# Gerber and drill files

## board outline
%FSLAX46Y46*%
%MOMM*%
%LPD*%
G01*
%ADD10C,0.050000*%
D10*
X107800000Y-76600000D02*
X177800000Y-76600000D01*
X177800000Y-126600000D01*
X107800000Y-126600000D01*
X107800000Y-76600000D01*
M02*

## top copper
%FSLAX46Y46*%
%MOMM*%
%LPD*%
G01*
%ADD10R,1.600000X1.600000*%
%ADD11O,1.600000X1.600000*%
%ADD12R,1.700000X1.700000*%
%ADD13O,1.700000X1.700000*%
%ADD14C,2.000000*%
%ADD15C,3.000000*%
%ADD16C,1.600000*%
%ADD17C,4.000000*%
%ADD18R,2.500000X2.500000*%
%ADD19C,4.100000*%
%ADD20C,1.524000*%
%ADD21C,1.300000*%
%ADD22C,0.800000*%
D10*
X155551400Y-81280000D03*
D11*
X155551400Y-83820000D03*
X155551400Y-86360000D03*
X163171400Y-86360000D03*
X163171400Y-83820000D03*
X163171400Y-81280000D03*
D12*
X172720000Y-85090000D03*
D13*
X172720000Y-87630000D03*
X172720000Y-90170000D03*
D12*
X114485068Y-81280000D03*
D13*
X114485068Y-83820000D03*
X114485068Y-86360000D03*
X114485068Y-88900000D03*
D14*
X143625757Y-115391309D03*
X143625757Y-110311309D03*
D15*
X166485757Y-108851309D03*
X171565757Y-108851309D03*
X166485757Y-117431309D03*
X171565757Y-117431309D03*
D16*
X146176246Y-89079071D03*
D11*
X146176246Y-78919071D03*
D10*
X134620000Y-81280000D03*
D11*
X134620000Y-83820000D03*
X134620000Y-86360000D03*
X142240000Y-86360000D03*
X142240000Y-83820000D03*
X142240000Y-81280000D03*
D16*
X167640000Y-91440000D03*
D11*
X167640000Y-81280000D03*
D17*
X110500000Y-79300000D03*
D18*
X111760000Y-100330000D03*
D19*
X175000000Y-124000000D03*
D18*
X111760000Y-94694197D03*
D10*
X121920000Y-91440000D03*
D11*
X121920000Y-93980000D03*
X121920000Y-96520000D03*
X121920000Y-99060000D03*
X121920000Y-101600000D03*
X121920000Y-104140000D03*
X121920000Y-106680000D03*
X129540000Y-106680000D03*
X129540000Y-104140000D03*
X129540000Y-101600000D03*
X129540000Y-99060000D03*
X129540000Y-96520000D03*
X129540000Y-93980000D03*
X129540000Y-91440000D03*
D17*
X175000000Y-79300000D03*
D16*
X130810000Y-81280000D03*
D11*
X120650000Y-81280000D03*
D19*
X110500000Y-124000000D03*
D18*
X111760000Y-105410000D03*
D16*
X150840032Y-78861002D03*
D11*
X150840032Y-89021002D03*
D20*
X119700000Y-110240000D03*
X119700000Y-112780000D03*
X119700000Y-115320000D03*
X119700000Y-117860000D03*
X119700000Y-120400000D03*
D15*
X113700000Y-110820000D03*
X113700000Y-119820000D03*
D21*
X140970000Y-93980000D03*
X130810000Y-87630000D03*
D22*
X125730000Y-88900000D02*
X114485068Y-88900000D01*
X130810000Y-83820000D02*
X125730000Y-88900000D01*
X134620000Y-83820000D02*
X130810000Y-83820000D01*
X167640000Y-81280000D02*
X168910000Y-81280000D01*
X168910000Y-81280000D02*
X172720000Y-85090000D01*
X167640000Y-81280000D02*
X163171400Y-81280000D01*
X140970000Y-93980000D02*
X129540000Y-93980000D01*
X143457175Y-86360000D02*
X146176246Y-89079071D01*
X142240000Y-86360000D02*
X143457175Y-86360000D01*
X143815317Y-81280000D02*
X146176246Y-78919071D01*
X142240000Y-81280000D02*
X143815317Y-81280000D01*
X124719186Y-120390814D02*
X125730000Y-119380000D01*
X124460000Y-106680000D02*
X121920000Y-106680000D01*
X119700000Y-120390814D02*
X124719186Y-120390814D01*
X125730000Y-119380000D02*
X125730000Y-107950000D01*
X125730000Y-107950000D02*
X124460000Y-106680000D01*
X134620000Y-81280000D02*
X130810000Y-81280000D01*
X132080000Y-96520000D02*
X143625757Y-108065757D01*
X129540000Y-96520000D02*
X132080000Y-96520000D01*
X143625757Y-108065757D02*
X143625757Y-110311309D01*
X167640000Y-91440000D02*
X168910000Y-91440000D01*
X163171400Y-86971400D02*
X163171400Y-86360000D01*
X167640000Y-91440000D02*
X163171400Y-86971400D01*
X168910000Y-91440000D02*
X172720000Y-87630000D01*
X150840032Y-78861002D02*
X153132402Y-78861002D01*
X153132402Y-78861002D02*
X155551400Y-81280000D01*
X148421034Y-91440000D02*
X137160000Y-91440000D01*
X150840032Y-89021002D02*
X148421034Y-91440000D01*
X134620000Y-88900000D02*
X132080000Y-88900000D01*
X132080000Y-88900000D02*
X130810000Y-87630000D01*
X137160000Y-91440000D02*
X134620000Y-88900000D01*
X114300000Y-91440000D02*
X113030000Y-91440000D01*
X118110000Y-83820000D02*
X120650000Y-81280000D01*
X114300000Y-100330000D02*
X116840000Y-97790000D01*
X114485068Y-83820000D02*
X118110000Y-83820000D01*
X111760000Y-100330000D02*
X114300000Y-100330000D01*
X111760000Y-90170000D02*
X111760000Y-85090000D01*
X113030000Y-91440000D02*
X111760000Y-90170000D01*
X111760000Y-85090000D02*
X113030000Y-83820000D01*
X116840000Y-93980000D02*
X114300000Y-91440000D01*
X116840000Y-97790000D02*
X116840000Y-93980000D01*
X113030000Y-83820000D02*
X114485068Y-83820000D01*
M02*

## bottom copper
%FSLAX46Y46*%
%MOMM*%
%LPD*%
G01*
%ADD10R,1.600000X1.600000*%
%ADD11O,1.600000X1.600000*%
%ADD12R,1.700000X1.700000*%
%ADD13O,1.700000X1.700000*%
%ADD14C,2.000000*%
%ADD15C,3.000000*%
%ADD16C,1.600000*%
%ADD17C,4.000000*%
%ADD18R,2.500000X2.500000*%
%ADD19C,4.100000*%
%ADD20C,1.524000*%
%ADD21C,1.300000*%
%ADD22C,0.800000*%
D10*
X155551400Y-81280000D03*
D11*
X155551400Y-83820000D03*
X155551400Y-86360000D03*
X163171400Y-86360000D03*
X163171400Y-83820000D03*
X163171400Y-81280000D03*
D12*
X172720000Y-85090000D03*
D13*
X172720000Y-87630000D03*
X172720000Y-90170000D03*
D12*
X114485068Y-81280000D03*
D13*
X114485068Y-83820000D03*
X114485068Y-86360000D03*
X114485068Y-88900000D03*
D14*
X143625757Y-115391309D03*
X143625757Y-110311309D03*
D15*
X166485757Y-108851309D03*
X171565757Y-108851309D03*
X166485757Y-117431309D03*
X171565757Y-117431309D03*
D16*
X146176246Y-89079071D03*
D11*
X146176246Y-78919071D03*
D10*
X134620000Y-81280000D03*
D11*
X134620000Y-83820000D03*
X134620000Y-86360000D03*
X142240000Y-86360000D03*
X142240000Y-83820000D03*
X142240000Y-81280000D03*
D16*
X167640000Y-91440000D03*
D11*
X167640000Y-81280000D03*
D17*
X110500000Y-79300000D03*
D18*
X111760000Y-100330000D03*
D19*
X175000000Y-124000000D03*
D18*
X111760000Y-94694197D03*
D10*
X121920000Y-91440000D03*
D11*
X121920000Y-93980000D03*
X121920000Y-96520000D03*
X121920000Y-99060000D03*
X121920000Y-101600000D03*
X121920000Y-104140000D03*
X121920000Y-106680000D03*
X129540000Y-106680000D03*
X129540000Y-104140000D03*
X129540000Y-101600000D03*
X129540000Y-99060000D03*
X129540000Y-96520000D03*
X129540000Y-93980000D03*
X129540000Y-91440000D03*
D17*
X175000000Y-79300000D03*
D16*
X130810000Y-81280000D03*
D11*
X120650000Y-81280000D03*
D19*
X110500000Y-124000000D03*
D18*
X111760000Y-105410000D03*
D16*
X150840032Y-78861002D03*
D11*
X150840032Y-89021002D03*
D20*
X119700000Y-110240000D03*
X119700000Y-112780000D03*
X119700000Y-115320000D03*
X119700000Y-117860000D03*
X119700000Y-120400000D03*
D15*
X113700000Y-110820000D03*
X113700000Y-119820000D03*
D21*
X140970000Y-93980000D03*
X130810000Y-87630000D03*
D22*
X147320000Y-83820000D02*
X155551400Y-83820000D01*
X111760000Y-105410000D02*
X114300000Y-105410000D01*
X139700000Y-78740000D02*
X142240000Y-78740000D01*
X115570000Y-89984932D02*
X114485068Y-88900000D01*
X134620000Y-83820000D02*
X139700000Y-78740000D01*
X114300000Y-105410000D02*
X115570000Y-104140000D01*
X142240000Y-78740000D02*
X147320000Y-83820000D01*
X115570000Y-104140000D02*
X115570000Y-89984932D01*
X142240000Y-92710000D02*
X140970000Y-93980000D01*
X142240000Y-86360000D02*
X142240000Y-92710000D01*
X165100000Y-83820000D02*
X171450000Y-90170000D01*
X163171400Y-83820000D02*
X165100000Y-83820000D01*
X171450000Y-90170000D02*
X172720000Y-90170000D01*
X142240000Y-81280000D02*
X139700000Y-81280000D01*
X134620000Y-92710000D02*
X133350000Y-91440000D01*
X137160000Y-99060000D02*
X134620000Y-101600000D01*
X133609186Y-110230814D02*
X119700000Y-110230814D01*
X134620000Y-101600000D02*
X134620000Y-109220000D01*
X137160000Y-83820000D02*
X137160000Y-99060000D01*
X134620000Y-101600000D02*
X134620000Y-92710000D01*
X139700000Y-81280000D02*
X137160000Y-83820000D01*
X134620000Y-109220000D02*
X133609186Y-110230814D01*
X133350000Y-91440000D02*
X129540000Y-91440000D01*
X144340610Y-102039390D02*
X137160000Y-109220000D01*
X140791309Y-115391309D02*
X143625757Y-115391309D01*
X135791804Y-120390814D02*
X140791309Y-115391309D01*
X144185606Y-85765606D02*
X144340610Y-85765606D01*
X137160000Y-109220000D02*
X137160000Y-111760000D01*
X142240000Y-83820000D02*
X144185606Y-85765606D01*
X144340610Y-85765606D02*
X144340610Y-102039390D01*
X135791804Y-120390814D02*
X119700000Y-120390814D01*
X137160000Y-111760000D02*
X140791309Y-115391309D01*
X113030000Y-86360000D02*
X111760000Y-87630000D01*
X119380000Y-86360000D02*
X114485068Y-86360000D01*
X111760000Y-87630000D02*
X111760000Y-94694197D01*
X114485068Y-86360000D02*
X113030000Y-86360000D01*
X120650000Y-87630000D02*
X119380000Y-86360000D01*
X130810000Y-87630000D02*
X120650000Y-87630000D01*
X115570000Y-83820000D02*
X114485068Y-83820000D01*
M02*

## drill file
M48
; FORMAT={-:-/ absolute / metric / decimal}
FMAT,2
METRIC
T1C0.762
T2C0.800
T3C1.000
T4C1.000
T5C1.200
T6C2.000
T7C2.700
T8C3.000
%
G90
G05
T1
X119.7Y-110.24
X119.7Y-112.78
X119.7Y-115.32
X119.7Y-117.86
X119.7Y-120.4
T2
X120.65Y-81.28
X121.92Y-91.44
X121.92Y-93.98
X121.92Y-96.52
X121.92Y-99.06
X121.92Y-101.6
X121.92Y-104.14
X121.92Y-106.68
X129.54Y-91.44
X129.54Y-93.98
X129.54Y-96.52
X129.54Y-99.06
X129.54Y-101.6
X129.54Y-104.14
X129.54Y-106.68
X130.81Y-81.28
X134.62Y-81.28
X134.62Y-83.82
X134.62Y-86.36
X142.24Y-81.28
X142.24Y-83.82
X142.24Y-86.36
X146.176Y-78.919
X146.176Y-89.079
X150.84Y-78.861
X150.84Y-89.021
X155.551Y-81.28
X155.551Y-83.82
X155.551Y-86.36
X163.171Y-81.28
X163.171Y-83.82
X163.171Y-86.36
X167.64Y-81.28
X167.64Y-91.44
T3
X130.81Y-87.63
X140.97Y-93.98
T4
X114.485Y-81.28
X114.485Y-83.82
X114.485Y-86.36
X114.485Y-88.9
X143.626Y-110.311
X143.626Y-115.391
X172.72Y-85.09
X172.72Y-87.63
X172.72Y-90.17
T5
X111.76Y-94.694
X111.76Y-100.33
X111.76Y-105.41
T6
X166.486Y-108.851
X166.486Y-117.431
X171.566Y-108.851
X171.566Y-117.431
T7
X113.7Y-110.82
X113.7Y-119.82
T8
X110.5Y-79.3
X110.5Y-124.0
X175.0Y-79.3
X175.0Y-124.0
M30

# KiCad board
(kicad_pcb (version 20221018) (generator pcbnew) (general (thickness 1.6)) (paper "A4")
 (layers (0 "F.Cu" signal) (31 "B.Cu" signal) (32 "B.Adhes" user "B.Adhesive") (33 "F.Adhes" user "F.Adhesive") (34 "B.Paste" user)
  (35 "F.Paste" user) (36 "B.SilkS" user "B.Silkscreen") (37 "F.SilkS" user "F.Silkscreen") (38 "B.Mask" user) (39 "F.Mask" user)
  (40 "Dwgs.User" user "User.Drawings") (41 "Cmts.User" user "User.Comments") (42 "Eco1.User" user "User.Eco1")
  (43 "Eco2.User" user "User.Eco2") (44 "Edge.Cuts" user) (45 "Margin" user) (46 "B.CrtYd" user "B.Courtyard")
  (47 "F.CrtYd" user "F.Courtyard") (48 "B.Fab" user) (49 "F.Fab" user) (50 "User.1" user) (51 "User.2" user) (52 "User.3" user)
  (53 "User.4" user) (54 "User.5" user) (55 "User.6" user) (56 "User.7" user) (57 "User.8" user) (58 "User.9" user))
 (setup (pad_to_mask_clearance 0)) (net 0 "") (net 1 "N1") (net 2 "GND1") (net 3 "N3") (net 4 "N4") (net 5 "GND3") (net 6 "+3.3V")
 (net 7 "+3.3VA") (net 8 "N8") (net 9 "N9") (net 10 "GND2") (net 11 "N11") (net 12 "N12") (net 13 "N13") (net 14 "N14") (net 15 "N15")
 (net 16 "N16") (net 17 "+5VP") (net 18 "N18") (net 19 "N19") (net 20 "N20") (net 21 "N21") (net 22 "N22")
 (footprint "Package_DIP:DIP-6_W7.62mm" (layer "F.Cu") (at 155.5514 81.28)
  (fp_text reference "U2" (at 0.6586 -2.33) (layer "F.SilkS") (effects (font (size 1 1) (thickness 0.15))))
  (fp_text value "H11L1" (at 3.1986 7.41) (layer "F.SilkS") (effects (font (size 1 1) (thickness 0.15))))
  (pad "1" thru_hole rect (at 0 0) (size 1.6 1.6) (drill 0.8) (layers "*.Cu" "*.Mask") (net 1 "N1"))
  (pad "2" thru_hole oval (at 0 2.54) (size 1.6 1.6) (drill 0.8) (layers "*.Cu" "*.Mask") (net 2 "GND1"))
  (pad "3" thru_hole oval (at 0 5.08) (size 1.6 1.6) (drill 0.8) (layers "*.Cu" "*.Mask") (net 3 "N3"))
  (pad "4" thru_hole oval (at 7.62 5.08) (size 1.6 1.6) (drill 0.8) (layers "*.Cu" "*.Mask") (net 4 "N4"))
  (pad "5" thru_hole oval (at 7.62 2.54) (size 1.6 1.6) (drill 0.8) (layers "*.Cu" "*.Mask") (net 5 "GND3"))
  (pad "6" thru_hole oval (at 7.62 0) (size 1.6 1.6) (drill 0.8) (layers "*.Cu" "*.Mask") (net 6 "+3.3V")))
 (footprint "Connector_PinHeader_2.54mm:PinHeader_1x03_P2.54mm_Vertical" (layer "F.Cu") (at 172.72 85.09)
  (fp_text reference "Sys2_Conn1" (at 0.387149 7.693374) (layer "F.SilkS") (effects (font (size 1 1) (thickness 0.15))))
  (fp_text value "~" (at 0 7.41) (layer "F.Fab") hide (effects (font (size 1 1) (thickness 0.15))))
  (pad "1" thru_hole rect (at 0 0) (size 1.7 1.7) (drill 1) (layers "*.Cu" "*.Mask") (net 6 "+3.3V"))
  (pad "2" thru_hole oval (at 0 2.54) (size 1.7 1.7) (drill 1) (layers "*.Cu" "*.Mask") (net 4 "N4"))
  (pad "3" thru_hole oval (at 0 5.08) (size 1.7 1.7) (drill 1) (layers "*.Cu" "*.Mask") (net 5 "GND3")))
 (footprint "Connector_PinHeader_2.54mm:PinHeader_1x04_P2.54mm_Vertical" (layer "F.Cu") (at 114.485068 81.28)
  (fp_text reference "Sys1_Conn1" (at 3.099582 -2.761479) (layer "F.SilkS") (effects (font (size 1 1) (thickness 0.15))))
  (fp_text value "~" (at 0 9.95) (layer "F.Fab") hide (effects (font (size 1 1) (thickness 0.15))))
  (pad "1" thru_hole rect (at 0 0) (size 1.7 1.7) (drill 1) (layers "*.Cu" "*.Mask") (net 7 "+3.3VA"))
  (pad "2" thru_hole oval (at 0 2.54) (size 1.7 1.7) (drill 1) (layers "*.Cu" "*.Mask") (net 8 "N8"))
  (pad "3" thru_hole oval (at 0 5.08) (size 1.7 1.7) (drill 1) (layers "*.Cu" "*.Mask") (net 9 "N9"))
  (pad "4" thru_hole oval (at 0 7.62) (size 1.7 1.7) (drill 1) (layers "*.Cu" "*.Mask") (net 2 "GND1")))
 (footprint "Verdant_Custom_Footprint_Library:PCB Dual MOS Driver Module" (layer "F.Cu") (at 148.705757 112.851309)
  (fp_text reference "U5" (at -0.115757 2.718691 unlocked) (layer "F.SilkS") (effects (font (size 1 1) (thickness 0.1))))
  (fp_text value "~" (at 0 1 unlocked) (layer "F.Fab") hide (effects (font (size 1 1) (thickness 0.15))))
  (pad "1" thru_hole circle (at -5.08 2.54) (size 2 2) (drill 1) (layers "*.Cu" "*.Mask") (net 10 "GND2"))
  (pad "2" thru_hole circle (at -5.08 -2.54) (size 2 2) (drill 1) (layers "*.Cu" "*.Mask") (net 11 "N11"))
  (pad "3" thru_hole circle (at 17.78 -4 90) (size 3 3) (drill 2) (layers "*.Cu" "*.Mask") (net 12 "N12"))
  (pad "4" thru_hole circle (at 22.86 -4) (size 3 3) (drill 2) (layers "*.Cu" "*.Mask") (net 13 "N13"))
  (pad "5" thru_hole circle (at 17.78 4.58) (size 3 3) (drill 2) (layers "*.Cu" "*.Mask") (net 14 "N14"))
  (pad "6" thru_hole circle (at 22.86 4.58) (size 3 3) (drill 2) (layers "*.Cu" "*.Mask") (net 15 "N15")))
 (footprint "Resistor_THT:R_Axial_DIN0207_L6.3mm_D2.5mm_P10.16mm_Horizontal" (layer "F.Cu") (at 146.176246 89.079071 90)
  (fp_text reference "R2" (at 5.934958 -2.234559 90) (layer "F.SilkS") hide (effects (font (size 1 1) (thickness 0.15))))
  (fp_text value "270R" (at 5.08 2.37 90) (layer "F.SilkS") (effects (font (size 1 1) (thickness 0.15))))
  (pad "1" thru_hole circle (at 0 0 90) (size 1.6 1.6) (drill 0.8) (layers "*.Cu" "*.Mask") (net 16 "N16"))
  (pad "2" thru_hole oval (at 10.16 0 90) (size 1.6 1.6) (drill 0.8) (layers "*.Cu" "*.Mask") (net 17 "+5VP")))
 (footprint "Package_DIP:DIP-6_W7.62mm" (layer "F.Cu") (at 134.62 81.28)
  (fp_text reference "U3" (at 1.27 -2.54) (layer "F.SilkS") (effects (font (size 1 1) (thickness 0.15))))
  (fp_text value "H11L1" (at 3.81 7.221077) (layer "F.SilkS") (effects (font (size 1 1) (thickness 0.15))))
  (pad "1" thru_hole rect (at 0 0) (size 1.6 1.6) (drill 0.8) (layers "*.Cu" "*.Mask") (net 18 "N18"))
  (pad "2" thru_hole oval (at 0 2.54) (size 1.6 1.6) (drill 0.8) (layers "*.Cu" "*.Mask") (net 2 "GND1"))
  (pad "3" thru_hole oval (at 0 5.08) (size 1.6 1.6) (drill 0.8) (layers "*.Cu" "*.Mask") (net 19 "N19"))
  (pad "4" thru_hole oval (at 7.62 5.08) (size 1.6 1.6) (drill 0.8) (layers "*.Cu" "*.Mask") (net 16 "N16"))
  (pad "5" thru_hole oval (at 7.62 2.54) (size 1.6 1.6) (drill 0.8) (layers "*.Cu" "*.Mask") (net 10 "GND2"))
  (pad "6" thru_hole oval (at 7.62 0) (size 1.6 1.6) (drill 0.8) (layers "*.Cu" "*.Mask") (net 17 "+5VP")))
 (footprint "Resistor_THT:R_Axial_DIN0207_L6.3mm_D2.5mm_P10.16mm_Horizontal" (layer "F.Cu") (at 167.64 91.44 90)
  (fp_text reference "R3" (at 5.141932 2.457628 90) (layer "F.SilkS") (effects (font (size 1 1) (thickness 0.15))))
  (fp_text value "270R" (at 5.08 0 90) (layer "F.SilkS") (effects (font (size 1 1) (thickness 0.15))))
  (pad "1" thru_hole circle (at 0 0 90) (size 1.6 1.6) (drill 0.8) (layers "*.Cu" "*.Mask") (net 4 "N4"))
  (pad "2" thru_hole oval (at 10.16 0 90) (size 1.6 1.6) (drill 0.8) (layers "*.Cu" "*.Mask") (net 6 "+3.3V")))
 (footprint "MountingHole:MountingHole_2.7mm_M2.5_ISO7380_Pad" (layer "F.Cu") (at 110.5 79.3)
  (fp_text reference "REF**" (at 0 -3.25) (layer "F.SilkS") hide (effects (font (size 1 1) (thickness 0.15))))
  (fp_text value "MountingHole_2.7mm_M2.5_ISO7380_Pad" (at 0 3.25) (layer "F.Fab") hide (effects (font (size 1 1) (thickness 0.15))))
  (pad "1" thru_hole circle (at 0 0) (size 4 4) (drill 3) (layers "*.Cu" "*.Mask")))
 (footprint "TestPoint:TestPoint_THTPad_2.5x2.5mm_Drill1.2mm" (layer "F.Cu") (at 111.76 100.33)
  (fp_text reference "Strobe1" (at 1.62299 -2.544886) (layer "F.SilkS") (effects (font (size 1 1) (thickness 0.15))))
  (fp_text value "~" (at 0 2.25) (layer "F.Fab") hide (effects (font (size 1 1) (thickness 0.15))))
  (pad "1" thru_hole rect (at 0 0) (size 2.5 2.5) (drill 1.2) (layers "*.Cu" "*.Mask") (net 8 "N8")))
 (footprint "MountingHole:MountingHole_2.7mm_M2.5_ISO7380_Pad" (layer "F.Cu") (at 175 124)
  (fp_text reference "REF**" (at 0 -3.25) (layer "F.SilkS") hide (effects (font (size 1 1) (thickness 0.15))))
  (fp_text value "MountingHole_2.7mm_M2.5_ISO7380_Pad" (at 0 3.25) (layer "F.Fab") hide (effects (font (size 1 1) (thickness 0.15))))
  (pad "1" thru_hole circle (at 0 0) (size 4.1 4.1) (drill 3) (layers "*.Cu" "*.Mask")))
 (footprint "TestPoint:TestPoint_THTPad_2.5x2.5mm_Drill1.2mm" (layer "F.Cu") (at 111.76 94.694197)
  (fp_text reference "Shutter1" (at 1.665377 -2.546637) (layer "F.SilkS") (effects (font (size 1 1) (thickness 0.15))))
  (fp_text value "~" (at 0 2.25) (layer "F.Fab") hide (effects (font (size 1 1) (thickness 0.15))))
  (pad "1" thru_hole rect (at 0 0) (size 2.5 2.5) (drill 1.2) (layers "*.Cu" "*.Mask") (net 9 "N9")))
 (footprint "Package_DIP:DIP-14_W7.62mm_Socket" (layer "F.Cu") (at 121.92 91.44)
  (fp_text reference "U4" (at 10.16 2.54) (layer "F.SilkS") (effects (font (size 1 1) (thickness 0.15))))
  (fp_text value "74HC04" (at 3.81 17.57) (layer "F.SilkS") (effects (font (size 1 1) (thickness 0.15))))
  (pad "1" thru_hole rect (at 0 0) (size 1.6 1.6) (drill 0.8) (layers "*.Cu" "*.Mask"))
  (pad "2" thru_hole oval (at 0 2.54) (size 1.6 1.6) (drill 0.8) (layers "*.Cu" "*.Mask"))
  (pad "3" thru_hole oval (at 0 5.08) (size 1.6 1.6) (drill 0.8) (layers "*.Cu" "*.Mask"))
  (pad "4" thru_hole oval (at 0 7.62) (size 1.6 1.6) (drill 0.8) (layers "*.Cu" "*.Mask"))
  (pad "5" thru_hole oval (at 0 10.16) (size 1.6 1.6) (drill 0.8) (layers "*.Cu" "*.Mask"))
  (pad "6" thru_hole oval (at 0 12.7) (size 1.6 1.6) (drill 0.8) (layers "*.Cu" "*.Mask"))
  (pad "7" thru_hole oval (at 0 15.24) (size 1.6 1.6) (drill 0.8) (layers "*.Cu" "*.Mask") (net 10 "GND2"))
  (pad "8" thru_hole oval (at 7.62 15.24) (size 1.6 1.6) (drill 0.8) (layers "*.Cu" "*.Mask"))
  (pad "9" thru_hole oval (at 7.62 12.7) (size 1.6 1.6) (drill 0.8) (layers "*.Cu" "*.Mask"))
  (pad "10" thru_hole oval (at 7.62 10.16) (size 1.6 1.6) (drill 0.8) (layers "*.Cu" "*.Mask"))
  (pad "11" thru_hole oval (at 7.62 7.62) (size 1.6 1.6) (drill 0.8) (layers "*.Cu" "*.Mask"))
  (pad "12" thru_hole oval (at 7.62 5.08) (size 1.6 1.6) (drill 0.8) (layers "*.Cu" "*.Mask") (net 11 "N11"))
  (pad "13" thru_hole oval (at 7.62 2.54) (size 1.6 1.6) (drill 0.8) (layers "*.Cu" "*.Mask") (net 16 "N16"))
  (pad "14" thru_hole oval (at 7.62 0) (size 1.6 1.6) (drill 0.8) (layers "*.Cu" "*.Mask") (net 17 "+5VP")))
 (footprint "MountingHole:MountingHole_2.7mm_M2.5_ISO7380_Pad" (layer "F.Cu") (at 175 79.3)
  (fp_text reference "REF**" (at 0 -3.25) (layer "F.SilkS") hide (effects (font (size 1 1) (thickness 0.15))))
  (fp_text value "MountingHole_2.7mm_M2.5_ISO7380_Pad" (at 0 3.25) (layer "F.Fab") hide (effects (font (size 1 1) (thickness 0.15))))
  (pad "1" thru_hole circle (at 0 0) (size 4 4) (drill 3) (layers "*.Cu" "*.Mask")))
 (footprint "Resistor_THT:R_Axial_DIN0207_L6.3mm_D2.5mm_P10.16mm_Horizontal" (layer "F.Cu") (at 130.81 81.28 180)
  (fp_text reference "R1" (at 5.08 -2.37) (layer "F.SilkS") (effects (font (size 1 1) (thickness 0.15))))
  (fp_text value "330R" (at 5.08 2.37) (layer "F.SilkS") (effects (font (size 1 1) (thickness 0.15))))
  (pad "1" thru_hole circle (at 0 0 180) (size 1.6 1.6) (drill 0.8) (layers "*.Cu" "*.Mask") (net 18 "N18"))
  (pad "2" thru_hole oval (at 10.16 0 180) (size 1.6 1.6) (drill 0.8) (layers "*.Cu" "*.Mask") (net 8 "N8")))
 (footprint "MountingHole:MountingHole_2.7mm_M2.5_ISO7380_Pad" (layer "F.Cu") (at 110.5 124)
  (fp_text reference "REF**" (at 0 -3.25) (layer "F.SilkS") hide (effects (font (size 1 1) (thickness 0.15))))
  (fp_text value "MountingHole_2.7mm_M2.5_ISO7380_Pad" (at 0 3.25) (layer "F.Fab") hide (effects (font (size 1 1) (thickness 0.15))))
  (pad "1" thru_hole circle (at 0 0) (size 4.1 4.1) (drill 3) (layers "*.Cu" "*.Mask")))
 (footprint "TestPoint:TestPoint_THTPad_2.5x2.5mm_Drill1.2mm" (layer "F.Cu") (at 111.76 105.41)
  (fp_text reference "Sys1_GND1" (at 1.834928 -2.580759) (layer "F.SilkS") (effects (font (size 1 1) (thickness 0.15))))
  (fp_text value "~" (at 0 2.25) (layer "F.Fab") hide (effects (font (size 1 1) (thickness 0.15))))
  (pad "1" thru_hole rect (at 0 0) (size 2.5 2.5) (drill 1.2) (layers "*.Cu" "*.Mask") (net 2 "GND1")))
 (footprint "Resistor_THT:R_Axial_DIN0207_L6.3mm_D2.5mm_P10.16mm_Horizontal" (layer "F.Cu") (at 150.840032 78.861002 -90)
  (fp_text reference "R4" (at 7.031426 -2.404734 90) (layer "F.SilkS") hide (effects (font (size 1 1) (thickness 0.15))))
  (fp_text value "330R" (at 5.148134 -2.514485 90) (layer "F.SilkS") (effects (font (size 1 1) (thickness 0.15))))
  (pad "1" thru_hole circle (at 0 0 270) (size 1.6 1.6) (drill 0.8) (layers "*.Cu" "*.Mask") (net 1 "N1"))
  (pad "2" thru_hole oval (at 10.16 0 270) (size 1.6 1.6) (drill 0.8) (layers "*.Cu" "*.Mask") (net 9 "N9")))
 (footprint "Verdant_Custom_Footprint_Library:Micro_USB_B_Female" (layer "F.Cu") (at 119.7 115.32)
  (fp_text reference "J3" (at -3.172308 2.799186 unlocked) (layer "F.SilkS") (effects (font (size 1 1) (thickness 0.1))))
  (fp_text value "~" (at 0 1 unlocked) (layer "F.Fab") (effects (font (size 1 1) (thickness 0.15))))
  (pad "1" thru_hole circle (at 0 -5.08) (size 1.524 1.524) (drill 0.762) (layers "*.Cu" "*.Mask") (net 17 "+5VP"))
  (pad "2" thru_hole circle (at 0 -2.54) (size 1.524 1.524) (drill 0.762) (layers "*.Cu" "*.Mask") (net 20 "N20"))
  (pad "3" thru_hole circle (at 0 0) (size 1.524 1.524) (drill 0.762) (layers "*.Cu" "*.Mask") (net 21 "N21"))
  (pad "4" thru_hole circle (at 0 2.54) (size 1.524 1.524) (drill 0.762) (layers "*.Cu" "*.Mask") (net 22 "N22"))
  (pad "5" thru_hole circle (at 0 5.08) (size 1.524 1.524) (drill 0.762) (layers "*.Cu" "*.Mask") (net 10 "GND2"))
  (pad "6" thru_hole circle (at -6 -4.5) (size 3 3) (drill 2.7) (layers "*.Cu" "*.Mask"))
  (pad "7" thru_hole circle (at -6 4.5) (size 3 3) (drill 2.7) (layers "*.Cu" "*.Mask")))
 (gr_rect (start 107.8 76.6) (end 177.8 126.6) (stroke (width 0.05) (type default)) (fill none) (layer "Edge.Cuts"))
 (segment (start 125.73 88.9) (end 114.485068 88.9) (width 0.8) (layer "F.Cu") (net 2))
 (segment (start 130.81 83.82) (end 125.73 88.9) (width 0.8) (layer "F.Cu") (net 2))
 (segment (start 134.62 83.82) (end 130.81 83.82) (width 0.8) (layer "F.Cu") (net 2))
 (segment (start 147.32 83.82) (end 155.5514 83.82) (width 0.8) (layer "B.Cu") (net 2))
 (segment (start 111.76 105.41) (end 114.3 105.41) (width 0.8) (layer "B.Cu") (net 2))
 (segment (start 139.7 78.74) (end 142.24 78.74) (width 0.8) (layer "B.Cu") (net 2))
 (segment (start 115.57 89.984932) (end 114.485068 88.9) (width 0.8) (layer "B.Cu") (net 2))
 (segment (start 134.62 83.82) (end 139.7 78.74) (width 0.8) (layer "B.Cu") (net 2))
 (segment (start 114.3 105.41) (end 115.57 104.14) (width 0.8) (layer "B.Cu") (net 2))
 (segment (start 142.24 78.74) (end 147.32 83.82) (width 0.8) (layer "B.Cu") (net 2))
 (segment (start 115.57 104.14) (end 115.57 89.984932) (width 0.8) (layer "B.Cu") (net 2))
 (segment (start 167.64 81.28) (end 168.91 81.28) (width 0.8) (layer "F.Cu") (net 6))
 (segment (start 168.91 81.28) (end 172.72 85.09) (width 0.8) (layer "F.Cu") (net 6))
 (segment (start 167.64 81.28) (end 163.1714 81.28) (width 0.8) (layer "F.Cu") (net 6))
 (segment (start 140.97 93.98) (end 129.54 93.98) (width 0.8) (layer "F.Cu") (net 16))
 (segment (start 143.457175 86.36) (end 146.176246 89.079071) (width 0.8) (layer "F.Cu") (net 16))
 (segment (start 142.24 86.36) (end 143.457175 86.36) (width 0.8) (layer "F.Cu") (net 16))
 (via (at 140.97 93.98) (size 1.3) (drill 1) (layers "F.Cu" "B.Cu") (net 16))
 (segment (start 142.24 92.71) (end 140.97 93.98) (width 0.8) (layer "B.Cu") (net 16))
 (segment (start 142.24 86.36) (end 142.24 92.71) (width 0.8) (layer "B.Cu") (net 16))
 (segment (start 165.1 83.82) (end 171.45 90.17) (width 0.8) (layer "B.Cu") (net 5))
 (segment (start 163.1714 83.82) (end 165.1 83.82) (width 0.8) (layer "B.Cu") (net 5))
 (segment (start 171.45 90.17) (end 172.72 90.17) (width 0.8) (layer "B.Cu") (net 5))
 (segment (start 143.815317 81.28) (end 146.176246 78.919071) (width 0.8) (layer "F.Cu") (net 17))
 (segment (start 142.24 81.28) (end 143.815317 81.28) (width 0.8) (layer "F.Cu") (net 17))
 (segment (start 142.24 81.28) (end 139.7 81.28) (width 0.8) (layer "B.Cu") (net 17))
 (segment (start 134.62 92.71) (end 133.35 91.44) (width 0.8) (layer "B.Cu") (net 17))
 (segment (start 137.16 99.06) (end 134.62 101.6) (width 0.8) (layer "B.Cu") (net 17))
 (segment (start 133.609186 110.230814) (end 119.7 110.230814) (width 0.8) (layer "B.Cu") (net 17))
 (segment (start 134.62 101.6) (end 134.62 109.22) (width 0.8) (layer "B.Cu") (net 17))
 (segment (start 137.16 83.82) (end 137.16 99.06) (width 0.8) (layer "B.Cu") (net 17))
 (segment (start 134.62 101.6) (end 134.62 92.71) (width 0.8) (layer "B.Cu") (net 17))
 (segment (start 139.7 81.28) (end 137.16 83.82) (width 0.8) (layer "B.Cu") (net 17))
 (segment (start 134.62 109.22) (end 133.609186 110.230814) (width 0.8) (layer "B.Cu") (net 17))
 (segment (start 133.35 91.44) (end 129.54 91.44) (width 0.8) (layer "B.Cu") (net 17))
 (segment (start 124.719186 120.390814) (end 125.73 119.38) (width 0.8) (layer "F.Cu") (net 10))
 (segment (start 124.46 106.68) (end 121.92 106.68) (width 0.8) (layer "F.Cu") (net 10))
 (segment (start 119.7 120.390814) (end 124.719186 120.390814) (width 0.8) (layer "F.Cu") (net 10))
 (segment (start 125.73 119.38) (end 125.73 107.95) (width 0.8) (layer "F.Cu") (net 10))
 (segment (start 125.73 107.95) (end 124.46 106.68) (width 0.8) (layer "F.Cu") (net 10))
 (segment (start 144.34061 102.03939) (end 137.16 109.22) (width 0.8) (layer "B.Cu") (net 10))
 (segment (start 140.791309 115.391309) (end 143.625757 115.391309) (width 0.8) (layer "B.Cu") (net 10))
 (segment (start 135.791804 120.390814) (end 140.791309 115.391309) (width 0.8) (layer "B.Cu") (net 10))
 (segment (start 144.185606 85.765606) (end 144.34061 85.765606) (width 0.8) (layer "B.Cu") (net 10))
 (segment (start 137.16 109.22) (end 137.16 111.76) (width 0.8) (layer "B.Cu") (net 10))
 (segment (start 142.24 83.82) (end 144.185606 85.765606) (width 0.8) (layer "B.Cu") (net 10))
 (segment (start 144.34061 85.765606) (end 144.34061 102.03939) (width 0.8) (layer "B.Cu") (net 10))
 (segment (start 135.791804 120.390814) (end 119.7 120.390814) (width 0.8) (layer "B.Cu") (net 10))
 (segment (start 137.16 111.76) (end 140.791309 115.391309) (width 0.8) (layer "B.Cu") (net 10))
 (segment (start 134.62 81.28) (end 130.81 81.28) (width 0.8) (layer "F.Cu") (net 18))
 (segment (start 132.08 96.52) (end 143.625757 108.065757) (width 0.8) (layer "F.Cu") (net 11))
 (segment (start 129.54 96.52) (end 132.08 96.52) (width 0.8) (layer "F.Cu") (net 11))
 (segment (start 143.625757 108.065757) (end 143.625757 110.311309) (width 0.8) (layer "F.Cu") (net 11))
 (segment (start 167.64 91.44) (end 168.91 91.44) (width 0.8) (layer "F.Cu") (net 4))
 (segment (start 163.1714 86.9714) (end 163.1714 86.36) (width 0.8) (layer "F.Cu") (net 4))
 (segment (start 167.64 91.44) (end 163.1714 86.9714) (width 0.8) (layer "F.Cu") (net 4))
 (segment (start 168.91 91.44) (end 172.72 87.63) (width 0.8) (layer "F.Cu") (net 4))
 (segment (start 150.840032 78.861002) (end 153.132402 78.861002) (width 0.8) (layer "F.Cu") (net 1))
 (segment (start 153.132402 78.861002) (end 155.5514 81.28) (width 0.8) (layer "F.Cu") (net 1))
 (segment (start 148.421034 91.44) (end 137.16 91.44) (width 0.8) (layer "F.Cu") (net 9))
 (segment (start 150.840032 89.021002) (end 148.421034 91.44) (width 0.8) (layer "F.Cu") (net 9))
 (segment (start 134.62 88.9) (end 132.08 88.9) (width 0.8) (layer "F.Cu") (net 9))
 (segment (start 132.08 88.9) (end 130.81 87.63) (width 0.8) (layer "F.Cu") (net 9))
 (segment (start 137.16 91.44) (end 134.62 88.9) (width 0.8) (layer "F.Cu") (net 9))
 (via (at 130.81 87.63) (size 1.3) (drill 1) (layers "F.Cu" "B.Cu") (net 9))
 (segment (start 113.03 86.36) (end 111.76 87.63) (width 0.8) (layer "B.Cu") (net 9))
 (segment (start 119.38 86.36) (end 114.485068 86.36) (width 0.8) (layer "B.Cu") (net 9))
 (segment (start 111.76 87.63) (end 111.76 94.694197) (width 0.8) (layer "B.Cu") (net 9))
 (segment (start 114.485068 86.36) (end 113.03 86.36) (width 0.8) (layer "B.Cu") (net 9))
 (segment (start 120.65 87.63) (end 119.38 86.36) (width 0.8) (layer "B.Cu") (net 9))
 (segment (start 130.81 87.63) (end 120.65 87.63) (width 0.8) (layer "B.Cu") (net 9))
 (segment (start 114.3 91.44) (end 113.03 91.44) (width 0.8) (layer "F.Cu") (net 8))
 (segment (start 118.11 83.82) (end 120.65 81.28) (width 0.8) (layer "F.Cu") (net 8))
 (segment (start 114.3 100.33) (end 116.84 97.79) (width 0.8) (layer "F.Cu") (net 8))
 (segment (start 114.485068 83.82) (end 118.11 83.82) (width 0.8) (layer "F.Cu") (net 8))
 (segment (start 111.76 100.33) (end 114.3 100.33) (width 0.8) (layer "F.Cu") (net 8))
 (segment (start 111.76 90.17) (end 111.76 85.09) (width 0.8) (layer "F.Cu") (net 8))
 (segment (start 113.03 91.44) (end 111.76 90.17) (width 0.8) (layer "F.Cu") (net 8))
 (segment (start 111.76 85.09) (end 113.03 83.82) (width 0.8) (layer "F.Cu") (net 8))
 (segment (start 116.84 93.98) (end 114.3 91.44) (width 0.8) (layer "F.Cu") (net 8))
 (segment (start 116.84 97.79) (end 116.84 93.98) (width 0.8) (layer "F.Cu") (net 8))
 (segment (start 113.03 83.82) (end 114.485068 83.82) (width 0.8) (layer "F.Cu") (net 8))
 (segment (start 115.57 83.82) (end 114.485068 83.82) (width 0.8) (layer "B.Cu") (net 8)))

